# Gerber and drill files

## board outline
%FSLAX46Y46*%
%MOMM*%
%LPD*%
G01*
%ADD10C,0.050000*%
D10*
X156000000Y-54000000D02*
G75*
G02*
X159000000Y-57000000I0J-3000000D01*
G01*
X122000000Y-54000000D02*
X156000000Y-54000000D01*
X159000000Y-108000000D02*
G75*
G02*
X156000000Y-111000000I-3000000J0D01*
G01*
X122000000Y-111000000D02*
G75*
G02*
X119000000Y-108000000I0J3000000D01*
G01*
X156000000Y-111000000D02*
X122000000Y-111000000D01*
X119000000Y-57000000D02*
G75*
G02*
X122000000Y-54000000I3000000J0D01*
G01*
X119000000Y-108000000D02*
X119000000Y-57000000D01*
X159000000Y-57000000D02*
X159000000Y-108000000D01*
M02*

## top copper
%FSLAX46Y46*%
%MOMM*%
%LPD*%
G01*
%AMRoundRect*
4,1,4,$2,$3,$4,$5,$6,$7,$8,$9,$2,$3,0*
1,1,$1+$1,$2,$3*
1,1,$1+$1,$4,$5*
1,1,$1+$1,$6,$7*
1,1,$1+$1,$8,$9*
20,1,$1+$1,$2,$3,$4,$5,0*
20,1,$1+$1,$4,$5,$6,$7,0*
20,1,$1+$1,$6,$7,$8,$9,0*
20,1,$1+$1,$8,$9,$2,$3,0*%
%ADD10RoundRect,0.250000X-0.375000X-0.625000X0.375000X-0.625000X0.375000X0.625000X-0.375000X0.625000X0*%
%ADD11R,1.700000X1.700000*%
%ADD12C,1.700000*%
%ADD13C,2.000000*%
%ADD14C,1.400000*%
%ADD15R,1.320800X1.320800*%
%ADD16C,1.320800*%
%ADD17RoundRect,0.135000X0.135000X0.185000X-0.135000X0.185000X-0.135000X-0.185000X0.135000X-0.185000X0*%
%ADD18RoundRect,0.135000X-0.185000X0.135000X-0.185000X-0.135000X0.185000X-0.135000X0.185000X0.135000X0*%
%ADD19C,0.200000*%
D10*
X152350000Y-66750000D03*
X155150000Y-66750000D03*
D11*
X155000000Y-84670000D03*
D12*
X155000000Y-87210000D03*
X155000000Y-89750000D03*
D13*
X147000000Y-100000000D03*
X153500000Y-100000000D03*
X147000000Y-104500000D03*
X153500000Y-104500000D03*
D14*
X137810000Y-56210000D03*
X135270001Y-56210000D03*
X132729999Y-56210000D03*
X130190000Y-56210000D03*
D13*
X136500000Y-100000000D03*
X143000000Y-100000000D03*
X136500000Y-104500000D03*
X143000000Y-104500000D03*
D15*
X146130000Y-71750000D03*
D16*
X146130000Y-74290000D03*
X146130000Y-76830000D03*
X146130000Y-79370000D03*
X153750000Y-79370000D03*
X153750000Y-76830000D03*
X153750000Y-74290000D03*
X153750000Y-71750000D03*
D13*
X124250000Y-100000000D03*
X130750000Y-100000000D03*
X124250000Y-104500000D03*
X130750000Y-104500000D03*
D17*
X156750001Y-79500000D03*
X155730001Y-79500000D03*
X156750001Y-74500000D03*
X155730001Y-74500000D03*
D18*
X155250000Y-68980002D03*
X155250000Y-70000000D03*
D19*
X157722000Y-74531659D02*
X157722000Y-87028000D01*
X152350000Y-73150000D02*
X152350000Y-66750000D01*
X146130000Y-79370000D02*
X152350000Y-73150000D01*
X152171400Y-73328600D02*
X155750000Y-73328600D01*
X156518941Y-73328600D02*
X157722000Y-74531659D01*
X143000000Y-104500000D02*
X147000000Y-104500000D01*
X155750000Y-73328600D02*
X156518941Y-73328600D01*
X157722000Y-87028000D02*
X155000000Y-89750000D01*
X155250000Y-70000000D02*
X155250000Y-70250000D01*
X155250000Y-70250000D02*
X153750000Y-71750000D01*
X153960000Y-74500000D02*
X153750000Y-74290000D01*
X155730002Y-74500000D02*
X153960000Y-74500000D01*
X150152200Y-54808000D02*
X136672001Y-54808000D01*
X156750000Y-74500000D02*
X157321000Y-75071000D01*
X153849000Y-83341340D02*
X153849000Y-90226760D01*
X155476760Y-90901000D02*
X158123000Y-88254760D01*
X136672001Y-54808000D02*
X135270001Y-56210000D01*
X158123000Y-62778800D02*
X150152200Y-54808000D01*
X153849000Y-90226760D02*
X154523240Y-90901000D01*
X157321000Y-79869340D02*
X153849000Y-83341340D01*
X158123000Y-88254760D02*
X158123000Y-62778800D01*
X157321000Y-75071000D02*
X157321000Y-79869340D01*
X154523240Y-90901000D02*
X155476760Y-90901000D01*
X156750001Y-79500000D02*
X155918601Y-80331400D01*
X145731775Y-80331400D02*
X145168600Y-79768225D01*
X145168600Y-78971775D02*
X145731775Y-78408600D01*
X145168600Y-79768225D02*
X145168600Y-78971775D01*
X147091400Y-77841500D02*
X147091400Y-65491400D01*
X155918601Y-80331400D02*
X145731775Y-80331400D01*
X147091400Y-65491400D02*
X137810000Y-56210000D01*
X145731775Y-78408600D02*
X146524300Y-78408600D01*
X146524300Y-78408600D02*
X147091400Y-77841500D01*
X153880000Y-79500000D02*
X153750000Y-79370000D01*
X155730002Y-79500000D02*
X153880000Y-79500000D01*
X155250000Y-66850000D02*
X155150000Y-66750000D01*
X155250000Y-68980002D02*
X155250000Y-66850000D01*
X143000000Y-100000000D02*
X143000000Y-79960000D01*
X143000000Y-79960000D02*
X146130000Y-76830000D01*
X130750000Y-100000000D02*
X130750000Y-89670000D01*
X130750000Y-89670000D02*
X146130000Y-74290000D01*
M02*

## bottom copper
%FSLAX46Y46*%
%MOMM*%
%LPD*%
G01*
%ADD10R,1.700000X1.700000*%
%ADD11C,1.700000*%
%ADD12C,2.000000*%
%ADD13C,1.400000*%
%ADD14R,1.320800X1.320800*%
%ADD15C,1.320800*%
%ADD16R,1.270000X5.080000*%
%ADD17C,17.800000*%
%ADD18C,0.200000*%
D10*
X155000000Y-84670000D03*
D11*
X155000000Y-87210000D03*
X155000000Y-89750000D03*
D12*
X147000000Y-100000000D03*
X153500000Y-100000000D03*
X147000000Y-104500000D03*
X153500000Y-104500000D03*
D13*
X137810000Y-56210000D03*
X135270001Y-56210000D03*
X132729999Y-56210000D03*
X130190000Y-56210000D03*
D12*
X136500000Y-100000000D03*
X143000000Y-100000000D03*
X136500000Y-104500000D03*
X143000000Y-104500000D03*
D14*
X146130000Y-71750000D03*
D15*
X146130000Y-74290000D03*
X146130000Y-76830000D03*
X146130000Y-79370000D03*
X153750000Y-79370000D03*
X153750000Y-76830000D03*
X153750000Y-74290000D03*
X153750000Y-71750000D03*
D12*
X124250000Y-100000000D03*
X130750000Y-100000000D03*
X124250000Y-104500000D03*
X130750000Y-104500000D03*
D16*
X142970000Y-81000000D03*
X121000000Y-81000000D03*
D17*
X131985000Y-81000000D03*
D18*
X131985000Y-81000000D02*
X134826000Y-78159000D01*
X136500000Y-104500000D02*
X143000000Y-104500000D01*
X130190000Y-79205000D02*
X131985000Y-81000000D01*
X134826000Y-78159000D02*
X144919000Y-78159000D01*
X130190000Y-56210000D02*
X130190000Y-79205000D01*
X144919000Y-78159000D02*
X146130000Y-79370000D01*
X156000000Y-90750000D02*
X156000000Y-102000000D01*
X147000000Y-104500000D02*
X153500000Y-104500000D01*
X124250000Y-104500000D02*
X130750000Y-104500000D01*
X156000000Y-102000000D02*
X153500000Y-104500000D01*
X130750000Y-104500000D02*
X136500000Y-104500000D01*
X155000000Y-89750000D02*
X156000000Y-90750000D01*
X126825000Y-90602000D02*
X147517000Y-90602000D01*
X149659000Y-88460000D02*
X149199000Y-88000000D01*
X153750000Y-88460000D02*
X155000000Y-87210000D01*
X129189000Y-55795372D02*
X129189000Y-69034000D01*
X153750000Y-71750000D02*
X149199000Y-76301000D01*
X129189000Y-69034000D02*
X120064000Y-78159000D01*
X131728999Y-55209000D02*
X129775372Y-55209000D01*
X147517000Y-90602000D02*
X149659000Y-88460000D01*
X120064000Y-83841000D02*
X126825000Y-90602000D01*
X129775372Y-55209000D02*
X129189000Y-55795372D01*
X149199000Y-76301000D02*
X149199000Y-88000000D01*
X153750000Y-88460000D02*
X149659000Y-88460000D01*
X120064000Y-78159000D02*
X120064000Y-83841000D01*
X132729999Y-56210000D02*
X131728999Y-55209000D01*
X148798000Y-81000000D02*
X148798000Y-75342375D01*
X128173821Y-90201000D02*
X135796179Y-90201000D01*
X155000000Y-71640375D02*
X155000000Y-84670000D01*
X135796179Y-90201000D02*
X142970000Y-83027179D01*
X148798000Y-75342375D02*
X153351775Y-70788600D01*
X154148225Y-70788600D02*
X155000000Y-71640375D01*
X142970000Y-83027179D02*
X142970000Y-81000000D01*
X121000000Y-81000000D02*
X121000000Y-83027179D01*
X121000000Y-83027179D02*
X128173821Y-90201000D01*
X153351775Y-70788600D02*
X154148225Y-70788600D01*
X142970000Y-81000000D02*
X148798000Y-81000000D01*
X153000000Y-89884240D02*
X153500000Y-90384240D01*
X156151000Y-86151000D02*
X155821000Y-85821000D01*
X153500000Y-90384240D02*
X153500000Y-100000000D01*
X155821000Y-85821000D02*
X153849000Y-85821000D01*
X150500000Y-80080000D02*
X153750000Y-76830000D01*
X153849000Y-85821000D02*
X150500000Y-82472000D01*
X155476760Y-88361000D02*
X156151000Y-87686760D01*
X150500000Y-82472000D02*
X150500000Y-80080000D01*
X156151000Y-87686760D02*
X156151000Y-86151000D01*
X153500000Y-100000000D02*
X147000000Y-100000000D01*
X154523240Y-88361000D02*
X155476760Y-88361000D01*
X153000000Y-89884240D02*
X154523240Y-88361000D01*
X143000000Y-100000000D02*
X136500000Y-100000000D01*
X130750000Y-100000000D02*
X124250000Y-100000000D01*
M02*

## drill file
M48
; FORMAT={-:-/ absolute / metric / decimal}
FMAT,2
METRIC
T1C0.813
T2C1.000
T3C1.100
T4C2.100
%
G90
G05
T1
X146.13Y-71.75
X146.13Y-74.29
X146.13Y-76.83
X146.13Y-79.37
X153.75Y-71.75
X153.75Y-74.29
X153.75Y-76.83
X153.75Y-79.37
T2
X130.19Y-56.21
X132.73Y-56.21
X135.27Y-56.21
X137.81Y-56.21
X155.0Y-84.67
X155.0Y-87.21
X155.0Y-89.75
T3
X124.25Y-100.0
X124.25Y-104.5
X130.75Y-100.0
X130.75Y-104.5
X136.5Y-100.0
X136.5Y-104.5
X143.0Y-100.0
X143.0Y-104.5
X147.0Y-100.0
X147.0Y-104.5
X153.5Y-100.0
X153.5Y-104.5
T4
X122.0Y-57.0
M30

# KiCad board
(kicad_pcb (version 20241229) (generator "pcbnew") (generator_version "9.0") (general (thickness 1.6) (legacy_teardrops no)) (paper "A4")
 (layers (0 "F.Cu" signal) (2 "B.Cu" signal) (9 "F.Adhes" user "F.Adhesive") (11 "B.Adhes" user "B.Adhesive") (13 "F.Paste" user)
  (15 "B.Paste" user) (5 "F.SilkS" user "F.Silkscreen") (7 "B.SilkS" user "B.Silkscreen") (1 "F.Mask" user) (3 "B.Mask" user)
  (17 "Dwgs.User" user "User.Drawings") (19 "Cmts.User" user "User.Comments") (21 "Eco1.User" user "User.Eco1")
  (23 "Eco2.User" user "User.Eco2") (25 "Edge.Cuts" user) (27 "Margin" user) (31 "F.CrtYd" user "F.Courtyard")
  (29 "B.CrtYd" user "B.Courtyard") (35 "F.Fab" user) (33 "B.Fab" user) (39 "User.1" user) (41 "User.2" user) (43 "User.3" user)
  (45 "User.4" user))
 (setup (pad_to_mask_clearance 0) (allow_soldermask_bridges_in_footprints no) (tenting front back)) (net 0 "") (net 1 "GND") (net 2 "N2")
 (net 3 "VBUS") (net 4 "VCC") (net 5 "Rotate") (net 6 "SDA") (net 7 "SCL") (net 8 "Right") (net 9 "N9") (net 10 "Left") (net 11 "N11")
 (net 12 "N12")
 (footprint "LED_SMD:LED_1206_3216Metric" (layer "F.Cu") (at 153.75 66.75)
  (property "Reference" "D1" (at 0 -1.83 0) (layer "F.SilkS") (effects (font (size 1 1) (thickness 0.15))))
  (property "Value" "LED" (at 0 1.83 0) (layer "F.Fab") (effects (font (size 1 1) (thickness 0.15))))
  (pad "1" smd roundrect (at -1.4 0) (size 1.25 1.75) (layers "F.Cu" "F.Mask" "F.Paste") (roundrect_rratio 0.2) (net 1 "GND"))
  (pad "2" smd roundrect (at 1.4 0) (size 1.25 1.75) (layers "F.Cu" "F.Mask" "F.Paste") (roundrect_rratio 0.2) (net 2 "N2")))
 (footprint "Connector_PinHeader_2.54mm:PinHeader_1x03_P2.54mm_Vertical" (layer "F.Cu") (at 155 84.67)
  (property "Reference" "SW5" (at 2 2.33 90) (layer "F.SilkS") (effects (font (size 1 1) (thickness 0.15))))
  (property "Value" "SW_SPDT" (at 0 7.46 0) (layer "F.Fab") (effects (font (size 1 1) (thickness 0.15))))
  (pad "1" thru_hole rect (at 0 0) (size 1.7 1.7) (drill 1) (layers "*.Cu" "*.Mask") (remove_unused_layers no) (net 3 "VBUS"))
  (pad "2" thru_hole circle (at 0 2.54) (size 1.7 1.7) (drill 1) (layers "*.Cu" "*.Mask") (remove_unused_layers no) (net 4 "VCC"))
  (pad "3" thru_hole circle (at 0 5.08) (size 1.7 1.7) (drill 1) (layers "*.Cu" "*.Mask") (remove_unused_layers no) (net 1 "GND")))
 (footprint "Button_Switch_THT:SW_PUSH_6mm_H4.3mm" (layer "F.Cu") (at 147 100)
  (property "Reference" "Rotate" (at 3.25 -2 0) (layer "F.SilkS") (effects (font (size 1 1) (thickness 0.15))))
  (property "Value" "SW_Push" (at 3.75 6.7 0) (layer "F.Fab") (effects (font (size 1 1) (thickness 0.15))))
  (pad "1" thru_hole circle (at 0 0 90) (size 2 2) (drill 1.1) (layers "*.Cu" "*.Mask") (remove_unused_layers no) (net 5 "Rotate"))
  (pad "1" thru_hole circle (at 6.5 0 90) (size 2 2) (drill 1.1) (layers "*.Cu" "*.Mask") (remove_unused_layers no) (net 5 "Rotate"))
  (pad "2" thru_hole circle (at 0 4.5 90) (size 2 2) (drill 1.1) (layers "*.Cu" "*.Mask") (remove_unused_layers no) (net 1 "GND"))
  (pad "2" thru_hole circle (at 6.5 4.5 90) (size 2 2) (drill 1.1) (layers "*.Cu" "*.Mask") (remove_unused_layers no) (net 1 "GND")))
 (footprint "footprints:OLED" (layer "F.Cu") (at 134 56.21 180)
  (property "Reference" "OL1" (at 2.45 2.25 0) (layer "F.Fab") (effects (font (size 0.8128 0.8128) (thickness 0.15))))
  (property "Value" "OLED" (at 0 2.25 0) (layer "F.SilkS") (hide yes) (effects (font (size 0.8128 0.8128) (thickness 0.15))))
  (pad "1" thru_hole circle (at -3.81 0 180) (size 1.4 1.4) (drill 1) (layers "*.Cu" "*.Mask") (remove_unused_layers no) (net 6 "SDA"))
  (pad "2" thru_hole circle (at -1.270001 0 180) (size 1.4 1.4) (drill 1) (layers "*.Cu" "*.Mask") (remove_unused_layers no) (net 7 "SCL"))
  (pad "3" thru_hole circle (at 1.270001 0 180) (size 1.4 1.4) (drill 1) (layers "*.Cu" "*.Mask") (remove_unused_layers no) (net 4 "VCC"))
  (pad "4" thru_hole circle (at 3.81 0 180) (size 1.4 1.4) (drill 1) (layers "*.Cu" "*.Mask") (remove_unused_layers no) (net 1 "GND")))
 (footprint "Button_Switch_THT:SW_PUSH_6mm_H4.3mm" (layer "F.Cu") (at 136.5 100)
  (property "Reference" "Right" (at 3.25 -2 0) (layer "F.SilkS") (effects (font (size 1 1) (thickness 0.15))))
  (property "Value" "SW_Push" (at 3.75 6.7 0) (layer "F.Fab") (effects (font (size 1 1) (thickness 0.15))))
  (pad "1" thru_hole circle (at 0 0 90) (size 2 2) (drill 1.1) (layers "*.Cu" "*.Mask") (remove_unused_layers no) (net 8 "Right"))
  (pad "1" thru_hole circle (at 6.5 0 90) (size 2 2) (drill 1.1) (layers "*.Cu" "*.Mask") (remove_unused_layers no) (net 8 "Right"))
  (pad "2" thru_hole circle (at 0 4.5 90) (size 2 2) (drill 1.1) (layers "*.Cu" "*.Mask") (remove_unused_layers no) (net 1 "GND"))
  (pad "2" thru_hole circle (at 6.5 4.5 90) (size 2 2) (drill 1.1) (layers "*.Cu" "*.Mask") (remove_unused_layers no) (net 1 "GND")))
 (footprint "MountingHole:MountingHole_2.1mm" (layer "F.Cu") (at 122 57)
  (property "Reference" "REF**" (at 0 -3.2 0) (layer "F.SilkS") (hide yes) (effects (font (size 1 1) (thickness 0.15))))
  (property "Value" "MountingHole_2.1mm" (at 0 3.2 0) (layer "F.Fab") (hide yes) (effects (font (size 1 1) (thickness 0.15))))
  (pad "" np_thru_hole circle (at 0 0) (size 2.1 2.1) (drill 2.1) (layers "*.Cu" "*.Mask")))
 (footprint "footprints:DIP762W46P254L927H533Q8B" (layer "F.Cu") (at 149.94 75.56)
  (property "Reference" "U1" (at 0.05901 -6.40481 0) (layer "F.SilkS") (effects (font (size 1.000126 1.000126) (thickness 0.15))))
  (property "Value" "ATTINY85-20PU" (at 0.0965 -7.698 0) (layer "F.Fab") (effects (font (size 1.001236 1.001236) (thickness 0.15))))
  (pad "1" thru_hole rect (at -3.81 -3.81) (size 1.3208 1.3208) (drill 0.8128) (layers "*.Cu" "*.Mask") (remove_unused_layers no)
   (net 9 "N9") (solder_mask_margin 0.102))
  (pad "2" thru_hole circle (at -3.81 -1.27) (size 1.3208 1.3208) (drill 0.8128) (layers "*.Cu" "*.Mask") (remove_unused_layers no)
   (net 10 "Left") (solder_mask_margin 0.102))
  (pad "3" thru_hole circle (at -3.81 1.27) (size 1.3208 1.3208) (drill 0.8128) (layers "*.Cu" "*.Mask") (remove_unused_layers no)
   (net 8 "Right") (solder_mask_margin 0.102))
  (pad "4" thru_hole circle (at -3.81 3.81) (size 1.3208 1.3208) (drill 0.8128) (layers "*.Cu" "*.Mask") (remove_unused_layers no)
   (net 1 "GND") (solder_mask_margin 0.102))
  (pad "5" thru_hole circle (at 3.81 3.81) (size 1.3208 1.3208) (drill 0.8128) (layers "*.Cu" "*.Mask") (remove_unused_layers no)
   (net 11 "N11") (solder_mask_margin 0.102))
  (pad "6" thru_hole circle (at 3.81 1.27) (size 1.3208 1.3208) (drill 0.8128) (layers "*.Cu" "*.Mask") (remove_unused_layers no)
   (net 5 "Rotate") (solder_mask_margin 0.102))
  (pad "7" thru_hole circle (at 3.81 -1.27) (size 1.3208 1.3208) (drill 0.8128) (layers "*.Cu" "*.Mask") (remove_unused_layers no)
   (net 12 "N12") (solder_mask_margin 0.102))
  (pad "8" thru_hole circle (at 3.81 -3.81) (size 1.3208 1.3208) (drill 0.8128) (layers "*.Cu" "*.Mask") (remove_unused_layers no)
   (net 4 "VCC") (solder_mask_margin 0.102)))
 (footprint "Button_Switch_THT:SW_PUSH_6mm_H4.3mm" (layer "F.Cu") (at 124.25 100)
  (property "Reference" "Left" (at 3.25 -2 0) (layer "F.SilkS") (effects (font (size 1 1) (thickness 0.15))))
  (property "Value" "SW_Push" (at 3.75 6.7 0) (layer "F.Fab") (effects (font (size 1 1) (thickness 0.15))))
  (pad "1" thru_hole circle (at 0 0 90) (size 2 2) (drill 1.1) (layers "*.Cu" "*.Mask") (remove_unused_layers no) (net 10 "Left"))
  (pad "1" thru_hole circle (at 6.5 0 90) (size 2 2) (drill 1.1) (layers "*.Cu" "*.Mask") (remove_unused_layers no) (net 10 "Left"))
  (pad "2" thru_hole circle (at 0 4.5 90) (size 2 2) (drill 1.1) (layers "*.Cu" "*.Mask") (remove_unused_layers no) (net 1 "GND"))
  (pad "2" thru_hole circle (at 6.5 4.5 90) (size 2 2) (drill 1.1) (layers "*.Cu" "*.Mask") (remove_unused_layers no) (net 1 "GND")))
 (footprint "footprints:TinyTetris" (layer "F.Cu") (at 147 89)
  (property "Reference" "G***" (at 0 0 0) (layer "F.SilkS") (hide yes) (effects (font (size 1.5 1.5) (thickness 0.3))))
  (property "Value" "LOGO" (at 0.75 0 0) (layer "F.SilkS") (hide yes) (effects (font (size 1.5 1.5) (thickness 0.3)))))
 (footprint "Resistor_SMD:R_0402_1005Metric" (layer "F.Cu") (at 156.240001 79.5 180)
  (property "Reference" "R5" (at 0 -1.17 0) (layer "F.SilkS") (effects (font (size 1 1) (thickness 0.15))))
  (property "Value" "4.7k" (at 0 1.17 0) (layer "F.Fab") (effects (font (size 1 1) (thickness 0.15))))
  (pad "1" smd roundrect (at -0.51 0 180) (size 0.54 0.64) (layers "F.Cu" "F.Mask" "F.Paste") (roundrect_rratio 0.25) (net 6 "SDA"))
  (pad "2" smd roundrect (at 0.51 0 180) (size 0.54 0.64) (layers "F.Cu" "F.Mask" "F.Paste") (roundrect_rratio 0.25) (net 11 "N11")))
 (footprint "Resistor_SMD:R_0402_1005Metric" (layer "F.Cu") (at 156.240001 74.5 180)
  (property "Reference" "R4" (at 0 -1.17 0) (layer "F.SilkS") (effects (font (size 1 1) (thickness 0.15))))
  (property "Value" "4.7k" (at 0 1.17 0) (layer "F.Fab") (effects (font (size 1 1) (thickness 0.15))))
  (pad "1" smd roundrect (at -0.51 0 180) (size 0.54 0.64) (layers "F.Cu" "F.Mask" "F.Paste") (roundrect_rratio 0.25) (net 7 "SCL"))
  (pad "2" smd roundrect (at 0.51 0 180) (size 0.54 0.64) (layers "F.Cu" "F.Mask" "F.Paste") (roundrect_rratio 0.25) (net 12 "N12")))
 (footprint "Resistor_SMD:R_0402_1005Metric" (layer "F.Cu") (at 155.25 69.490001 -90)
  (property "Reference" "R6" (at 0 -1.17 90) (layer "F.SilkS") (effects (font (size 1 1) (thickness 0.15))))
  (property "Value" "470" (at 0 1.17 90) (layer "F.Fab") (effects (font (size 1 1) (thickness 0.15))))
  (pad "1" smd roundrect (at -0.509999 0 270) (size 0.54 0.64) (layers "F.Cu" "F.Mask" "F.Paste") (roundrect_rratio 0.25) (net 2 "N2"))
  (pad "2" smd roundrect (at 0.509999 0 270) (size 0.54 0.64) (layers "F.Cu" "F.Mask" "F.Paste") (roundrect_rratio 0.25) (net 4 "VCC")))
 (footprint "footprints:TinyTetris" (layer "B.Cu") (at 147 89 180)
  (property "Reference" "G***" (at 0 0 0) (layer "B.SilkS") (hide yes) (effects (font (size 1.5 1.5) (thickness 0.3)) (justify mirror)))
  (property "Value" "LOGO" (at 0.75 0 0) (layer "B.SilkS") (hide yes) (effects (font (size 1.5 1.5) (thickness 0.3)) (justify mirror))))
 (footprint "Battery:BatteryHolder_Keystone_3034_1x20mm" (layer "B.Cu") (at 131.985 81 180)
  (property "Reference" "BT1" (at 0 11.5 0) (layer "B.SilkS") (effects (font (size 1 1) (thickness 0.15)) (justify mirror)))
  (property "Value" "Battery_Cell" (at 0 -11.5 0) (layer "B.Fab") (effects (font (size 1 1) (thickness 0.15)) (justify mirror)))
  (pad "1" smd rect (at -10.985 0 180) (size 1.27 5.08) (layers "B.Cu" "B.Mask" "B.Paste") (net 3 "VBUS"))
  (pad "1" smd rect (at 10.985 0 180) (size 1.27 5.08) (layers "B.Cu" "B.Mask" "B.Paste") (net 3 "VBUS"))
  (pad "2" smd circle (at 0 0 180) (size 17.8 17.8) (layers "B.Cu" "B.Mask") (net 1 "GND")))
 (gr_arc (start 156 54) (mid 158.12132 54.87868) (end 159 57) (stroke (width 0.05) (type default)) (layer "Edge.Cuts"))
 (gr_line (start 122 54) (end 156 54) (stroke (width 0.05) (type default)) (layer "Edge.Cuts"))
 (gr_arc (start 159 108) (mid 158.12132 110.12132) (end 156 111) (stroke (width 0.05) (type default)) (layer "Edge.Cuts"))
 (gr_arc (start 122 111) (mid 119.87868 110.12132) (end 119 108) (stroke (width 0.05) (type default)) (layer "Edge.Cuts"))
 (gr_line (start 156 111) (end 122 111) (stroke (width 0.05) (type default)) (layer "Edge.Cuts"))
 (gr_arc (start 119 57) (mid 119.87868 54.87868) (end 122 54) (stroke (width 0.05) (type default)) (layer "Edge.Cuts"))
 (gr_line (start 119 108) (end 119 57) (stroke (width 0.05) (type default)) (layer "Edge.Cuts"))
 (gr_line (start 159 57) (end 159 108) (stroke (width 0.05) (type default)) (layer "Edge.Cuts"))
 (segment (start 157.722 74.531659) (end 157.722 87.028) (width 0.2) (layer "F.Cu") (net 1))
 (segment (start 152.35 73.15) (end 152.35 66.75) (width 0.2) (layer "F.Cu") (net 1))
 (segment (start 146.13 79.37) (end 152.35 73.15) (width 0.2) (layer "F.Cu") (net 1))
 (segment (start 152.1714 73.3286) (end 155.75 73.3286) (width 0.2) (layer "F.Cu") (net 1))
 (segment (start 156.518941 73.3286) (end 157.722 74.531659) (width 0.2) (layer "F.Cu") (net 1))
 (segment (start 143 104.5) (end 147 104.5) (width 0.2) (layer "F.Cu") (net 1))
 (segment (start 155.75 73.3286) (end 156.518941 73.3286) (width 0.2) (layer "F.Cu") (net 1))
 (segment (start 157.722 87.028) (end 155 89.75) (width 0.2) (layer "F.Cu") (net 1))
 (segment (start 131.985 81) (end 134.826 78.159) (width 0.2) (layer "B.Cu") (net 1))
 (segment (start 136.5 104.5) (end 143 104.5) (width 0.2) (layer "B.Cu") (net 1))
 (segment (start 130.19 79.205) (end 131.985 81) (width 0.2) (layer "B.Cu") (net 1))
 (segment (start 134.826 78.159) (end 144.919 78.159) (width 0.2) (layer "B.Cu") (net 1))
 (segment (start 130.19 56.21) (end 130.19 79.205) (width 0.2) (layer "B.Cu") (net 1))
 (segment (start 144.919 78.159) (end 146.13 79.37) (width 0.2) (layer "B.Cu") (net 1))
 (segment (start 156 90.75) (end 156 102) (width 0.2) (layer "B.Cu") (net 1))
 (segment (start 147 104.5) (end 153.5 104.5) (width 0.2) (layer "B.Cu") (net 1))
 (segment (start 124.25 104.5) (end 130.75 104.5) (width 0.2) (layer "B.Cu") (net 1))
 (segment (start 156 102) (end 153.5 104.5) (width 0.2) (layer "B.Cu") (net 1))
 (segment (start 130.75 104.5) (end 136.5 104.5) (width 0.2) (layer "B.Cu") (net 1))
 (segment (start 155 89.75) (end 156 90.75) (width 0.2) (layer "B.Cu") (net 1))
 (segment (start 155.25 70) (end 155.25 70.25) (width 0.2) (layer "F.Cu") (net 4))
 (segment (start 155.25 70.25) (end 153.75 71.75) (width 0.2) (layer "F.Cu") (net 4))
 (segment (start 126.825 90.602) (end 147.517 90.602) (width 0.2) (layer "B.Cu") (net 4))
 (segment (start 149.659 88.46) (end 149.199 88) (width 0.2) (layer "B.Cu") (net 4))
 (segment (start 153.75 88.46) (end 155 87.21) (width 0.2) (layer "B.Cu") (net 4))
 (segment (start 129.189 55.795372) (end 129.189 69.034) (width 0.2) (layer "B.Cu") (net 4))
 (segment (start 153.75 71.75) (end 149.199 76.301) (width 0.2) (layer "B.Cu") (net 4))
 (segment (start 129.189 69.034) (end 120.064 78.159) (width 0.2) (layer "B.Cu") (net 4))
 (segment (start 131.728999 55.209) (end 129.775372 55.209) (width 0.2) (layer "B.Cu") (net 4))
 (segment (start 147.517 90.602) (end 149.659 88.46) (width 0.2) (layer "B.Cu") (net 4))
 (segment (start 120.064 83.841) (end 126.825 90.602) (width 0.2) (layer "B.Cu") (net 4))
 (segment (start 129.775372 55.209) (end 129.189 55.795372) (width 0.2) (layer "B.Cu") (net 4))
 (segment (start 149.199 76.301) (end 149.199 88) (width 0.2) (layer "B.Cu") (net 4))
 (segment (start 153.75 88.46) (end 149.659 88.46) (width 0.2) (layer "B.Cu") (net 4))
 (segment (start 120.064 78.159) (end 120.064 83.841) (width 0.2) (layer "B.Cu") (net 4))
 (segment (start 132.729999 56.21) (end 131.728999 55.209) (width 0.2) (layer "B.Cu") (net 4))
 (segment (start 153.96 74.5) (end 153.75 74.29) (width 0.2) (layer "F.Cu") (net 12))
 (segment (start 155.730002 74.5) (end 153.96 74.5) (width 0.2) (layer "F.Cu") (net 12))
 (segment (start 150.1522 54.808) (end 136.672001 54.808) (width 0.2) (layer "F.Cu") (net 7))
 (segment (start 156.75 74.5) (end 157.321 75.071) (width 0.2) (layer "F.Cu") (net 7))
 (segment (start 153.849 83.34134) (end 153.849 90.22676) (width 0.2) (layer "F.Cu") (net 7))
 (segment (start 155.47676 90.901) (end 158.123 88.25476) (width 0.2) (layer "F.Cu") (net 7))
 (segment (start 136.672001 54.808) (end 135.270001 56.21) (width 0.2) (layer "F.Cu") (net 7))
 (segment (start 158.123 62.7788) (end 150.1522 54.808) (width 0.2) (layer "F.Cu") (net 7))
 (segment (start 153.849 90.22676) (end 154.52324 90.901) (width 0.2) (layer "F.Cu") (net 7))
 (segment (start 157.321 79.86934) (end 153.849 83.34134) (width 0.2) (layer "F.Cu") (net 7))
 (segment (start 158.123 88.25476) (end 158.123 62.7788) (width 0.2) (layer "F.Cu") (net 7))
 (segment (start 157.321 75.071) (end 157.321 79.86934) (width 0.2) (layer "F.Cu") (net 7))
 (segment (start 154.52324 90.901) (end 155.47676 90.901) (width 0.2) (layer "F.Cu") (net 7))
 (segment (start 156.750001 79.5) (end 155.918601 80.3314) (width 0.2) (layer "F.Cu") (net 6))
 (segment (start 145.731775 80.3314) (end 145.1686 79.768225) (width 0.2) (layer "F.Cu") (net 6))
 (segment (start 145.1686 78.971775) (end 145.731775 78.4086) (width 0.2) (layer "F.Cu") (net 6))
 (segment (start 145.1686 79.768225) (end 145.1686 78.971775) (width 0.2) (layer "F.Cu") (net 6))
 (segment (start 147.0914 77.8415) (end 147.0914 65.4914) (width 0.2) (layer "F.Cu") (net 6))
 (segment (start 155.918601 80.3314) (end 145.731775 80.3314) (width 0.2) (layer "F.Cu") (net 6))
 (segment (start 147.0914 65.4914) (end 137.81 56.21) (width 0.2) (layer "F.Cu") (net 6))
 (segment (start 145.731775 78.4086) (end 146.5243 78.4086) (width 0.2) (layer "F.Cu") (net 6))
 (segment (start 146.5243 78.4086) (end 147.0914 77.8415) (width 0.2) (layer "F.Cu") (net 6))
 (segment (start 153.88 79.5) (end 153.75 79.37) (width 0.2) (layer "F.Cu") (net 11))
 (segment (start 155.730002 79.5) (end 153.88 79.5) (width 0.2) (layer "F.Cu") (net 11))
 (segment (start 148.798 81) (end 148.798 75.342375) (width 0.2) (layer "B.Cu") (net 3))
 (segment (start 128.173821 90.201) (end 135.796179 90.201) (width 0.2) (layer "B.Cu") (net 3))
 (segment (start 155 71.640375) (end 155 84.67) (width 0.2) (layer "B.Cu") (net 3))
 (segment (start 135.796179 90.201) (end 142.97 83.027179) (width 0.2) (layer "B.Cu") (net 3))
 (segment (start 148.798 75.342375) (end 153.351775 70.7886) (width 0.2) (layer "B.Cu") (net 3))
 (segment (start 154.148225 70.7886) (end 155 71.640375) (width 0.2) (layer "B.Cu") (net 3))
 (segment (start 142.97 83.027179) (end 142.97 81) (width 0.2) (layer "B.Cu") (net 3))
 (segment (start 121 81) (end 121 83.027179) (width 0.2) (layer "B.Cu") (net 3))
 (segment (start 121 83.027179) (end 128.173821 90.201) (width 0.2) (layer "B.Cu") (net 3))
 (segment (start 153.351775 70.7886) (end 154.148225 70.7886) (width 0.2) (layer "B.Cu") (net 3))
 (segment (start 142.97 81) (end 148.798 81) (width 0.2) (layer "B.Cu") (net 3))
 (segment (start 155.25 66.85) (end 155.15 66.75) (width 0.2) (layer "F.Cu") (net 2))
 (segment (start 155.25 68.980002) (end 155.25 66.85) (width 0.2) (layer "F.Cu") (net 2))
 (segment (start 153 89.88424) (end 153.5 90.38424) (width 0.2) (layer "B.Cu") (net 5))
 (segment (start 156.151 86.151) (end 155.821 85.821) (width 0.2) (layer "B.Cu") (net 5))
 (segment (start 153.5 90.38424) (end 153.5 100) (width 0.2) (layer "B.Cu") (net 5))
 (segment (start 155.821 85.821) (end 153.849 85.821) (width 0.2) (layer "B.Cu") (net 5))
 (segment (start 150.5 80.08) (end 153.75 76.83) (width 0.2) (layer "B.Cu") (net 5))
 (segment (start 153.849 85.821) (end 150.5 82.472) (width 0.2) (layer "B.Cu") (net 5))
 (segment (start 155.47676 88.361) (end 156.151 87.68676) (width 0.2) (layer "B.Cu") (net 5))
 (segment (start 150.5 82.472) (end 150.5 80.08) (width 0.2) (layer "B.Cu") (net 5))
 (segment (start 156.151 87.68676) (end 156.151 86.151) (width 0.2) (layer "B.Cu") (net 5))
 (segment (start 153.5 100) (end 147 100) (width 0.2) (layer "B.Cu") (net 5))
 (segment (start 154.52324 88.361) (end 155.47676 88.361) (width 0.2) (layer "B.Cu") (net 5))
 (segment (start 153 89.88424) (end 154.52324 88.361) (width 0.2) (layer "B.Cu") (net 5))
 (segment (start 143 100) (end 143 79.96) (width 0.2) (layer "F.Cu") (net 8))
 (segment (start 143 79.96) (end 146.13 76.83) (width 0.2) (layer "F.Cu") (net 8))
 (segment (start 143 100) (end 136.5 100) (width 0.2) (layer "B.Cu") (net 8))
 (segment (start 130.75 100) (end 130.75 89.67) (width 0.2) (layer "F.Cu") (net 10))
 (segment (start 130.75 89.67) (end 146.13 74.29) (width 0.2) (layer "F.Cu") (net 10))
 (segment (start 130.75 100) (end 124.25 100) (width 0.2) (layer "B.Cu") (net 10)))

